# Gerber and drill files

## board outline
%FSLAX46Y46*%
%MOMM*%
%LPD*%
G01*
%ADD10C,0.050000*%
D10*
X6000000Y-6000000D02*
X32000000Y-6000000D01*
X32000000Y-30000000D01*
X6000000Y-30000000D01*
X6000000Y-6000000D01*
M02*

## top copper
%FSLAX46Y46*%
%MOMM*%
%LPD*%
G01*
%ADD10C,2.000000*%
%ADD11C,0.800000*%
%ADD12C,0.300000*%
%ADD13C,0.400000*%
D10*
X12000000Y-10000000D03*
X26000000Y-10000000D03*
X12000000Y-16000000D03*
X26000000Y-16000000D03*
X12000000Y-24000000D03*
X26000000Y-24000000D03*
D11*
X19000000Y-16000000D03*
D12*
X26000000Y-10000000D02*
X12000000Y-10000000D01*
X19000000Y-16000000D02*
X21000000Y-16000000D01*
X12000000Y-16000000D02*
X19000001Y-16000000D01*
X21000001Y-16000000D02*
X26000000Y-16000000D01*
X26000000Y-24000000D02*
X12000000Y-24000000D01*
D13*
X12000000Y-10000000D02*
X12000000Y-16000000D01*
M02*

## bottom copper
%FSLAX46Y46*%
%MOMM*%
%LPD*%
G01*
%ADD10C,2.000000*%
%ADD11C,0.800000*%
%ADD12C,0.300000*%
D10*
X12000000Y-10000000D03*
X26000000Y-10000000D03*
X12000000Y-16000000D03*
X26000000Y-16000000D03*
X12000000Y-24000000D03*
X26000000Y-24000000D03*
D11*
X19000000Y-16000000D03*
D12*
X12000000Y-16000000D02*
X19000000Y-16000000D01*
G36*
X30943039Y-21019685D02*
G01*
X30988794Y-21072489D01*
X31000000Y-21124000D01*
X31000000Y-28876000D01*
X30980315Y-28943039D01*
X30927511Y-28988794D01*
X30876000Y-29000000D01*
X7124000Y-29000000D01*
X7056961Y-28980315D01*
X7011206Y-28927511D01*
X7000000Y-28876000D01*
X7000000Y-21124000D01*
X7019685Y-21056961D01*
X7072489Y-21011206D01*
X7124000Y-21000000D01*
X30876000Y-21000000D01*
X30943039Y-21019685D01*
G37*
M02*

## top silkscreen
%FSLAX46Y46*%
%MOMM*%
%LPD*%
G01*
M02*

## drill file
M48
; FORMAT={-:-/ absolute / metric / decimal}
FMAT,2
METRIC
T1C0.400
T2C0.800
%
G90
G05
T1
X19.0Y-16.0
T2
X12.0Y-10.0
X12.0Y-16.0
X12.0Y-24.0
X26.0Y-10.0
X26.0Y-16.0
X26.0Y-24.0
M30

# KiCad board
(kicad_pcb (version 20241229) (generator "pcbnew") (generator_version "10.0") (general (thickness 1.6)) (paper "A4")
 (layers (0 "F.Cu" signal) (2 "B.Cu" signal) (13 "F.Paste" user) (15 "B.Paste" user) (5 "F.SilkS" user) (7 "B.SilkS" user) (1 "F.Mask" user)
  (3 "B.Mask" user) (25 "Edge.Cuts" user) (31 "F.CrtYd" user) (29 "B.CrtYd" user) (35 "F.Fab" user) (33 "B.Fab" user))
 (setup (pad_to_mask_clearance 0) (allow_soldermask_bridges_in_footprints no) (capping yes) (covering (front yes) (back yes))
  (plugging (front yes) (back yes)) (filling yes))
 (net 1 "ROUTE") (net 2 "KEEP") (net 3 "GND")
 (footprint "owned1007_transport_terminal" (layer "F.Cu") (at 12 10)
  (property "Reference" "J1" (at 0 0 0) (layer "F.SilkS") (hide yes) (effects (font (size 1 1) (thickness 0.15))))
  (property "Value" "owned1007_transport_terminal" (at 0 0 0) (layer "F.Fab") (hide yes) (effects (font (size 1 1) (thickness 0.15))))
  (pad "1" thru_hole circle (at 0 0) (size 2 2) (drill 0.8) (layers "*.Cu" "*.Mask") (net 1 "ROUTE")))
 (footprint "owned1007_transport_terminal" (layer "F.Cu") (at 26 10)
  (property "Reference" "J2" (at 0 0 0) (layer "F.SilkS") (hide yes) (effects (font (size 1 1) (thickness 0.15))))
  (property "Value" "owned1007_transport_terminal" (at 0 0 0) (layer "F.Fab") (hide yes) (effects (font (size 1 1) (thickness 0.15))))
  (pad "1" thru_hole circle (at 0 0) (size 2 2) (drill 0.8) (layers "*.Cu" "*.Mask") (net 1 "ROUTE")))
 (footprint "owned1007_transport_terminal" (layer "F.Cu") (at 12 16)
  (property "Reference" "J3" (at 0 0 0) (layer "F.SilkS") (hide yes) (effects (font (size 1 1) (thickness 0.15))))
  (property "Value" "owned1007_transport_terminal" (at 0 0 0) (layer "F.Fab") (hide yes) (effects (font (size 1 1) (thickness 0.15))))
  (pad "1" thru_hole circle (at 0 0) (size 2 2) (drill 0.8) (layers "*.Cu" "*.Mask") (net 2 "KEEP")))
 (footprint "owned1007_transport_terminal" (layer "F.Cu") (at 26 16)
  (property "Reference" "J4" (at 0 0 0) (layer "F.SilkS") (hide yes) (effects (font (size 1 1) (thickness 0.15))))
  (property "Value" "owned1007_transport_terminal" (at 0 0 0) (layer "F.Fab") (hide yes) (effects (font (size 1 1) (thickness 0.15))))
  (pad "1" thru_hole circle (at 0 0) (size 2 2) (drill 0.8) (layers "*.Cu" "*.Mask") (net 2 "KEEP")))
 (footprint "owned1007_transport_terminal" (layer "F.Cu") (at 12 24)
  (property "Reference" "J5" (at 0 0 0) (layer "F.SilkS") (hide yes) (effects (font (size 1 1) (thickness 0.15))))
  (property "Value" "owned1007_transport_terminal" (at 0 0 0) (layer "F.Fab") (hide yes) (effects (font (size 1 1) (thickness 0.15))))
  (pad "1" thru_hole circle (at 0 0) (size 2 2) (drill 0.8) (layers "*.Cu" "*.Mask") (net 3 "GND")))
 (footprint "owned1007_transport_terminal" (layer "F.Cu") (at 26 24)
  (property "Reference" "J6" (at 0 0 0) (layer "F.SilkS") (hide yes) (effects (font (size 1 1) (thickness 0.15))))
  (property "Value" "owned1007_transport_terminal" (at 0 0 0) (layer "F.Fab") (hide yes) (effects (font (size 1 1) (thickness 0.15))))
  (pad "1" thru_hole circle (at 0 0) (size 2 2) (drill 0.8) (layers "*.Cu" "*.Mask") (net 3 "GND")))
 (gr_rect (start 6 6) (end 32 30) (stroke (width 0.05) (type default)) (fill none) (layer "Edge.Cuts"))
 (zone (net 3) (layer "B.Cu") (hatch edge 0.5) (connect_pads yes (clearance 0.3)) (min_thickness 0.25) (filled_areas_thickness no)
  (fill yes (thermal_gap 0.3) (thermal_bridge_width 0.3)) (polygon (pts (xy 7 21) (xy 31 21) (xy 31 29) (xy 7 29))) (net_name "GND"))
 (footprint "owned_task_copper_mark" (layer "F.Cu") (at 10 28)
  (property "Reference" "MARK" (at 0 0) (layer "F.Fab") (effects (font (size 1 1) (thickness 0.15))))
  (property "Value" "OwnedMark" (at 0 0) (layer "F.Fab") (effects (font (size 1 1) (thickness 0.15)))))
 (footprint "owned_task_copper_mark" (layer "F.Cu") (at 13 28)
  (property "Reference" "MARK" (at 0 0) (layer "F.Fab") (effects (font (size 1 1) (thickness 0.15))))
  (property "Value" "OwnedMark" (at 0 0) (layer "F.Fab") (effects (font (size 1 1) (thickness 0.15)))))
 (segment (start 26 10) (end 12 10) (width 0.3) (layer "F.Cu") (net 1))
 (segment (start 19 16) (end 21 16) (width 0.3) (layer "F.Cu") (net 2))
 (segment (start 12 16) (end 19.000001 16) (width 0.3) (layer "F.Cu") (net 2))
 (segment (start 21.000001 16) (end 26 16) (width 0.3) (layer "F.Cu") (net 2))
 (via (at 19 16) (size 0.8) (drill 0.4) (layers "F.Cu" "B.Cu") (free yes) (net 2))
 (segment (start 12 16) (end 19 16) (width 0.3) (layer "B.Cu") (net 2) (locked yes))
 (segment (start 26 24) (end 12 24) (width 0.3) (layer "F.Cu") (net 3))
 (segment (start 12 10) (end 12 16) (width 0.4) (layer "F.Cu") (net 1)))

